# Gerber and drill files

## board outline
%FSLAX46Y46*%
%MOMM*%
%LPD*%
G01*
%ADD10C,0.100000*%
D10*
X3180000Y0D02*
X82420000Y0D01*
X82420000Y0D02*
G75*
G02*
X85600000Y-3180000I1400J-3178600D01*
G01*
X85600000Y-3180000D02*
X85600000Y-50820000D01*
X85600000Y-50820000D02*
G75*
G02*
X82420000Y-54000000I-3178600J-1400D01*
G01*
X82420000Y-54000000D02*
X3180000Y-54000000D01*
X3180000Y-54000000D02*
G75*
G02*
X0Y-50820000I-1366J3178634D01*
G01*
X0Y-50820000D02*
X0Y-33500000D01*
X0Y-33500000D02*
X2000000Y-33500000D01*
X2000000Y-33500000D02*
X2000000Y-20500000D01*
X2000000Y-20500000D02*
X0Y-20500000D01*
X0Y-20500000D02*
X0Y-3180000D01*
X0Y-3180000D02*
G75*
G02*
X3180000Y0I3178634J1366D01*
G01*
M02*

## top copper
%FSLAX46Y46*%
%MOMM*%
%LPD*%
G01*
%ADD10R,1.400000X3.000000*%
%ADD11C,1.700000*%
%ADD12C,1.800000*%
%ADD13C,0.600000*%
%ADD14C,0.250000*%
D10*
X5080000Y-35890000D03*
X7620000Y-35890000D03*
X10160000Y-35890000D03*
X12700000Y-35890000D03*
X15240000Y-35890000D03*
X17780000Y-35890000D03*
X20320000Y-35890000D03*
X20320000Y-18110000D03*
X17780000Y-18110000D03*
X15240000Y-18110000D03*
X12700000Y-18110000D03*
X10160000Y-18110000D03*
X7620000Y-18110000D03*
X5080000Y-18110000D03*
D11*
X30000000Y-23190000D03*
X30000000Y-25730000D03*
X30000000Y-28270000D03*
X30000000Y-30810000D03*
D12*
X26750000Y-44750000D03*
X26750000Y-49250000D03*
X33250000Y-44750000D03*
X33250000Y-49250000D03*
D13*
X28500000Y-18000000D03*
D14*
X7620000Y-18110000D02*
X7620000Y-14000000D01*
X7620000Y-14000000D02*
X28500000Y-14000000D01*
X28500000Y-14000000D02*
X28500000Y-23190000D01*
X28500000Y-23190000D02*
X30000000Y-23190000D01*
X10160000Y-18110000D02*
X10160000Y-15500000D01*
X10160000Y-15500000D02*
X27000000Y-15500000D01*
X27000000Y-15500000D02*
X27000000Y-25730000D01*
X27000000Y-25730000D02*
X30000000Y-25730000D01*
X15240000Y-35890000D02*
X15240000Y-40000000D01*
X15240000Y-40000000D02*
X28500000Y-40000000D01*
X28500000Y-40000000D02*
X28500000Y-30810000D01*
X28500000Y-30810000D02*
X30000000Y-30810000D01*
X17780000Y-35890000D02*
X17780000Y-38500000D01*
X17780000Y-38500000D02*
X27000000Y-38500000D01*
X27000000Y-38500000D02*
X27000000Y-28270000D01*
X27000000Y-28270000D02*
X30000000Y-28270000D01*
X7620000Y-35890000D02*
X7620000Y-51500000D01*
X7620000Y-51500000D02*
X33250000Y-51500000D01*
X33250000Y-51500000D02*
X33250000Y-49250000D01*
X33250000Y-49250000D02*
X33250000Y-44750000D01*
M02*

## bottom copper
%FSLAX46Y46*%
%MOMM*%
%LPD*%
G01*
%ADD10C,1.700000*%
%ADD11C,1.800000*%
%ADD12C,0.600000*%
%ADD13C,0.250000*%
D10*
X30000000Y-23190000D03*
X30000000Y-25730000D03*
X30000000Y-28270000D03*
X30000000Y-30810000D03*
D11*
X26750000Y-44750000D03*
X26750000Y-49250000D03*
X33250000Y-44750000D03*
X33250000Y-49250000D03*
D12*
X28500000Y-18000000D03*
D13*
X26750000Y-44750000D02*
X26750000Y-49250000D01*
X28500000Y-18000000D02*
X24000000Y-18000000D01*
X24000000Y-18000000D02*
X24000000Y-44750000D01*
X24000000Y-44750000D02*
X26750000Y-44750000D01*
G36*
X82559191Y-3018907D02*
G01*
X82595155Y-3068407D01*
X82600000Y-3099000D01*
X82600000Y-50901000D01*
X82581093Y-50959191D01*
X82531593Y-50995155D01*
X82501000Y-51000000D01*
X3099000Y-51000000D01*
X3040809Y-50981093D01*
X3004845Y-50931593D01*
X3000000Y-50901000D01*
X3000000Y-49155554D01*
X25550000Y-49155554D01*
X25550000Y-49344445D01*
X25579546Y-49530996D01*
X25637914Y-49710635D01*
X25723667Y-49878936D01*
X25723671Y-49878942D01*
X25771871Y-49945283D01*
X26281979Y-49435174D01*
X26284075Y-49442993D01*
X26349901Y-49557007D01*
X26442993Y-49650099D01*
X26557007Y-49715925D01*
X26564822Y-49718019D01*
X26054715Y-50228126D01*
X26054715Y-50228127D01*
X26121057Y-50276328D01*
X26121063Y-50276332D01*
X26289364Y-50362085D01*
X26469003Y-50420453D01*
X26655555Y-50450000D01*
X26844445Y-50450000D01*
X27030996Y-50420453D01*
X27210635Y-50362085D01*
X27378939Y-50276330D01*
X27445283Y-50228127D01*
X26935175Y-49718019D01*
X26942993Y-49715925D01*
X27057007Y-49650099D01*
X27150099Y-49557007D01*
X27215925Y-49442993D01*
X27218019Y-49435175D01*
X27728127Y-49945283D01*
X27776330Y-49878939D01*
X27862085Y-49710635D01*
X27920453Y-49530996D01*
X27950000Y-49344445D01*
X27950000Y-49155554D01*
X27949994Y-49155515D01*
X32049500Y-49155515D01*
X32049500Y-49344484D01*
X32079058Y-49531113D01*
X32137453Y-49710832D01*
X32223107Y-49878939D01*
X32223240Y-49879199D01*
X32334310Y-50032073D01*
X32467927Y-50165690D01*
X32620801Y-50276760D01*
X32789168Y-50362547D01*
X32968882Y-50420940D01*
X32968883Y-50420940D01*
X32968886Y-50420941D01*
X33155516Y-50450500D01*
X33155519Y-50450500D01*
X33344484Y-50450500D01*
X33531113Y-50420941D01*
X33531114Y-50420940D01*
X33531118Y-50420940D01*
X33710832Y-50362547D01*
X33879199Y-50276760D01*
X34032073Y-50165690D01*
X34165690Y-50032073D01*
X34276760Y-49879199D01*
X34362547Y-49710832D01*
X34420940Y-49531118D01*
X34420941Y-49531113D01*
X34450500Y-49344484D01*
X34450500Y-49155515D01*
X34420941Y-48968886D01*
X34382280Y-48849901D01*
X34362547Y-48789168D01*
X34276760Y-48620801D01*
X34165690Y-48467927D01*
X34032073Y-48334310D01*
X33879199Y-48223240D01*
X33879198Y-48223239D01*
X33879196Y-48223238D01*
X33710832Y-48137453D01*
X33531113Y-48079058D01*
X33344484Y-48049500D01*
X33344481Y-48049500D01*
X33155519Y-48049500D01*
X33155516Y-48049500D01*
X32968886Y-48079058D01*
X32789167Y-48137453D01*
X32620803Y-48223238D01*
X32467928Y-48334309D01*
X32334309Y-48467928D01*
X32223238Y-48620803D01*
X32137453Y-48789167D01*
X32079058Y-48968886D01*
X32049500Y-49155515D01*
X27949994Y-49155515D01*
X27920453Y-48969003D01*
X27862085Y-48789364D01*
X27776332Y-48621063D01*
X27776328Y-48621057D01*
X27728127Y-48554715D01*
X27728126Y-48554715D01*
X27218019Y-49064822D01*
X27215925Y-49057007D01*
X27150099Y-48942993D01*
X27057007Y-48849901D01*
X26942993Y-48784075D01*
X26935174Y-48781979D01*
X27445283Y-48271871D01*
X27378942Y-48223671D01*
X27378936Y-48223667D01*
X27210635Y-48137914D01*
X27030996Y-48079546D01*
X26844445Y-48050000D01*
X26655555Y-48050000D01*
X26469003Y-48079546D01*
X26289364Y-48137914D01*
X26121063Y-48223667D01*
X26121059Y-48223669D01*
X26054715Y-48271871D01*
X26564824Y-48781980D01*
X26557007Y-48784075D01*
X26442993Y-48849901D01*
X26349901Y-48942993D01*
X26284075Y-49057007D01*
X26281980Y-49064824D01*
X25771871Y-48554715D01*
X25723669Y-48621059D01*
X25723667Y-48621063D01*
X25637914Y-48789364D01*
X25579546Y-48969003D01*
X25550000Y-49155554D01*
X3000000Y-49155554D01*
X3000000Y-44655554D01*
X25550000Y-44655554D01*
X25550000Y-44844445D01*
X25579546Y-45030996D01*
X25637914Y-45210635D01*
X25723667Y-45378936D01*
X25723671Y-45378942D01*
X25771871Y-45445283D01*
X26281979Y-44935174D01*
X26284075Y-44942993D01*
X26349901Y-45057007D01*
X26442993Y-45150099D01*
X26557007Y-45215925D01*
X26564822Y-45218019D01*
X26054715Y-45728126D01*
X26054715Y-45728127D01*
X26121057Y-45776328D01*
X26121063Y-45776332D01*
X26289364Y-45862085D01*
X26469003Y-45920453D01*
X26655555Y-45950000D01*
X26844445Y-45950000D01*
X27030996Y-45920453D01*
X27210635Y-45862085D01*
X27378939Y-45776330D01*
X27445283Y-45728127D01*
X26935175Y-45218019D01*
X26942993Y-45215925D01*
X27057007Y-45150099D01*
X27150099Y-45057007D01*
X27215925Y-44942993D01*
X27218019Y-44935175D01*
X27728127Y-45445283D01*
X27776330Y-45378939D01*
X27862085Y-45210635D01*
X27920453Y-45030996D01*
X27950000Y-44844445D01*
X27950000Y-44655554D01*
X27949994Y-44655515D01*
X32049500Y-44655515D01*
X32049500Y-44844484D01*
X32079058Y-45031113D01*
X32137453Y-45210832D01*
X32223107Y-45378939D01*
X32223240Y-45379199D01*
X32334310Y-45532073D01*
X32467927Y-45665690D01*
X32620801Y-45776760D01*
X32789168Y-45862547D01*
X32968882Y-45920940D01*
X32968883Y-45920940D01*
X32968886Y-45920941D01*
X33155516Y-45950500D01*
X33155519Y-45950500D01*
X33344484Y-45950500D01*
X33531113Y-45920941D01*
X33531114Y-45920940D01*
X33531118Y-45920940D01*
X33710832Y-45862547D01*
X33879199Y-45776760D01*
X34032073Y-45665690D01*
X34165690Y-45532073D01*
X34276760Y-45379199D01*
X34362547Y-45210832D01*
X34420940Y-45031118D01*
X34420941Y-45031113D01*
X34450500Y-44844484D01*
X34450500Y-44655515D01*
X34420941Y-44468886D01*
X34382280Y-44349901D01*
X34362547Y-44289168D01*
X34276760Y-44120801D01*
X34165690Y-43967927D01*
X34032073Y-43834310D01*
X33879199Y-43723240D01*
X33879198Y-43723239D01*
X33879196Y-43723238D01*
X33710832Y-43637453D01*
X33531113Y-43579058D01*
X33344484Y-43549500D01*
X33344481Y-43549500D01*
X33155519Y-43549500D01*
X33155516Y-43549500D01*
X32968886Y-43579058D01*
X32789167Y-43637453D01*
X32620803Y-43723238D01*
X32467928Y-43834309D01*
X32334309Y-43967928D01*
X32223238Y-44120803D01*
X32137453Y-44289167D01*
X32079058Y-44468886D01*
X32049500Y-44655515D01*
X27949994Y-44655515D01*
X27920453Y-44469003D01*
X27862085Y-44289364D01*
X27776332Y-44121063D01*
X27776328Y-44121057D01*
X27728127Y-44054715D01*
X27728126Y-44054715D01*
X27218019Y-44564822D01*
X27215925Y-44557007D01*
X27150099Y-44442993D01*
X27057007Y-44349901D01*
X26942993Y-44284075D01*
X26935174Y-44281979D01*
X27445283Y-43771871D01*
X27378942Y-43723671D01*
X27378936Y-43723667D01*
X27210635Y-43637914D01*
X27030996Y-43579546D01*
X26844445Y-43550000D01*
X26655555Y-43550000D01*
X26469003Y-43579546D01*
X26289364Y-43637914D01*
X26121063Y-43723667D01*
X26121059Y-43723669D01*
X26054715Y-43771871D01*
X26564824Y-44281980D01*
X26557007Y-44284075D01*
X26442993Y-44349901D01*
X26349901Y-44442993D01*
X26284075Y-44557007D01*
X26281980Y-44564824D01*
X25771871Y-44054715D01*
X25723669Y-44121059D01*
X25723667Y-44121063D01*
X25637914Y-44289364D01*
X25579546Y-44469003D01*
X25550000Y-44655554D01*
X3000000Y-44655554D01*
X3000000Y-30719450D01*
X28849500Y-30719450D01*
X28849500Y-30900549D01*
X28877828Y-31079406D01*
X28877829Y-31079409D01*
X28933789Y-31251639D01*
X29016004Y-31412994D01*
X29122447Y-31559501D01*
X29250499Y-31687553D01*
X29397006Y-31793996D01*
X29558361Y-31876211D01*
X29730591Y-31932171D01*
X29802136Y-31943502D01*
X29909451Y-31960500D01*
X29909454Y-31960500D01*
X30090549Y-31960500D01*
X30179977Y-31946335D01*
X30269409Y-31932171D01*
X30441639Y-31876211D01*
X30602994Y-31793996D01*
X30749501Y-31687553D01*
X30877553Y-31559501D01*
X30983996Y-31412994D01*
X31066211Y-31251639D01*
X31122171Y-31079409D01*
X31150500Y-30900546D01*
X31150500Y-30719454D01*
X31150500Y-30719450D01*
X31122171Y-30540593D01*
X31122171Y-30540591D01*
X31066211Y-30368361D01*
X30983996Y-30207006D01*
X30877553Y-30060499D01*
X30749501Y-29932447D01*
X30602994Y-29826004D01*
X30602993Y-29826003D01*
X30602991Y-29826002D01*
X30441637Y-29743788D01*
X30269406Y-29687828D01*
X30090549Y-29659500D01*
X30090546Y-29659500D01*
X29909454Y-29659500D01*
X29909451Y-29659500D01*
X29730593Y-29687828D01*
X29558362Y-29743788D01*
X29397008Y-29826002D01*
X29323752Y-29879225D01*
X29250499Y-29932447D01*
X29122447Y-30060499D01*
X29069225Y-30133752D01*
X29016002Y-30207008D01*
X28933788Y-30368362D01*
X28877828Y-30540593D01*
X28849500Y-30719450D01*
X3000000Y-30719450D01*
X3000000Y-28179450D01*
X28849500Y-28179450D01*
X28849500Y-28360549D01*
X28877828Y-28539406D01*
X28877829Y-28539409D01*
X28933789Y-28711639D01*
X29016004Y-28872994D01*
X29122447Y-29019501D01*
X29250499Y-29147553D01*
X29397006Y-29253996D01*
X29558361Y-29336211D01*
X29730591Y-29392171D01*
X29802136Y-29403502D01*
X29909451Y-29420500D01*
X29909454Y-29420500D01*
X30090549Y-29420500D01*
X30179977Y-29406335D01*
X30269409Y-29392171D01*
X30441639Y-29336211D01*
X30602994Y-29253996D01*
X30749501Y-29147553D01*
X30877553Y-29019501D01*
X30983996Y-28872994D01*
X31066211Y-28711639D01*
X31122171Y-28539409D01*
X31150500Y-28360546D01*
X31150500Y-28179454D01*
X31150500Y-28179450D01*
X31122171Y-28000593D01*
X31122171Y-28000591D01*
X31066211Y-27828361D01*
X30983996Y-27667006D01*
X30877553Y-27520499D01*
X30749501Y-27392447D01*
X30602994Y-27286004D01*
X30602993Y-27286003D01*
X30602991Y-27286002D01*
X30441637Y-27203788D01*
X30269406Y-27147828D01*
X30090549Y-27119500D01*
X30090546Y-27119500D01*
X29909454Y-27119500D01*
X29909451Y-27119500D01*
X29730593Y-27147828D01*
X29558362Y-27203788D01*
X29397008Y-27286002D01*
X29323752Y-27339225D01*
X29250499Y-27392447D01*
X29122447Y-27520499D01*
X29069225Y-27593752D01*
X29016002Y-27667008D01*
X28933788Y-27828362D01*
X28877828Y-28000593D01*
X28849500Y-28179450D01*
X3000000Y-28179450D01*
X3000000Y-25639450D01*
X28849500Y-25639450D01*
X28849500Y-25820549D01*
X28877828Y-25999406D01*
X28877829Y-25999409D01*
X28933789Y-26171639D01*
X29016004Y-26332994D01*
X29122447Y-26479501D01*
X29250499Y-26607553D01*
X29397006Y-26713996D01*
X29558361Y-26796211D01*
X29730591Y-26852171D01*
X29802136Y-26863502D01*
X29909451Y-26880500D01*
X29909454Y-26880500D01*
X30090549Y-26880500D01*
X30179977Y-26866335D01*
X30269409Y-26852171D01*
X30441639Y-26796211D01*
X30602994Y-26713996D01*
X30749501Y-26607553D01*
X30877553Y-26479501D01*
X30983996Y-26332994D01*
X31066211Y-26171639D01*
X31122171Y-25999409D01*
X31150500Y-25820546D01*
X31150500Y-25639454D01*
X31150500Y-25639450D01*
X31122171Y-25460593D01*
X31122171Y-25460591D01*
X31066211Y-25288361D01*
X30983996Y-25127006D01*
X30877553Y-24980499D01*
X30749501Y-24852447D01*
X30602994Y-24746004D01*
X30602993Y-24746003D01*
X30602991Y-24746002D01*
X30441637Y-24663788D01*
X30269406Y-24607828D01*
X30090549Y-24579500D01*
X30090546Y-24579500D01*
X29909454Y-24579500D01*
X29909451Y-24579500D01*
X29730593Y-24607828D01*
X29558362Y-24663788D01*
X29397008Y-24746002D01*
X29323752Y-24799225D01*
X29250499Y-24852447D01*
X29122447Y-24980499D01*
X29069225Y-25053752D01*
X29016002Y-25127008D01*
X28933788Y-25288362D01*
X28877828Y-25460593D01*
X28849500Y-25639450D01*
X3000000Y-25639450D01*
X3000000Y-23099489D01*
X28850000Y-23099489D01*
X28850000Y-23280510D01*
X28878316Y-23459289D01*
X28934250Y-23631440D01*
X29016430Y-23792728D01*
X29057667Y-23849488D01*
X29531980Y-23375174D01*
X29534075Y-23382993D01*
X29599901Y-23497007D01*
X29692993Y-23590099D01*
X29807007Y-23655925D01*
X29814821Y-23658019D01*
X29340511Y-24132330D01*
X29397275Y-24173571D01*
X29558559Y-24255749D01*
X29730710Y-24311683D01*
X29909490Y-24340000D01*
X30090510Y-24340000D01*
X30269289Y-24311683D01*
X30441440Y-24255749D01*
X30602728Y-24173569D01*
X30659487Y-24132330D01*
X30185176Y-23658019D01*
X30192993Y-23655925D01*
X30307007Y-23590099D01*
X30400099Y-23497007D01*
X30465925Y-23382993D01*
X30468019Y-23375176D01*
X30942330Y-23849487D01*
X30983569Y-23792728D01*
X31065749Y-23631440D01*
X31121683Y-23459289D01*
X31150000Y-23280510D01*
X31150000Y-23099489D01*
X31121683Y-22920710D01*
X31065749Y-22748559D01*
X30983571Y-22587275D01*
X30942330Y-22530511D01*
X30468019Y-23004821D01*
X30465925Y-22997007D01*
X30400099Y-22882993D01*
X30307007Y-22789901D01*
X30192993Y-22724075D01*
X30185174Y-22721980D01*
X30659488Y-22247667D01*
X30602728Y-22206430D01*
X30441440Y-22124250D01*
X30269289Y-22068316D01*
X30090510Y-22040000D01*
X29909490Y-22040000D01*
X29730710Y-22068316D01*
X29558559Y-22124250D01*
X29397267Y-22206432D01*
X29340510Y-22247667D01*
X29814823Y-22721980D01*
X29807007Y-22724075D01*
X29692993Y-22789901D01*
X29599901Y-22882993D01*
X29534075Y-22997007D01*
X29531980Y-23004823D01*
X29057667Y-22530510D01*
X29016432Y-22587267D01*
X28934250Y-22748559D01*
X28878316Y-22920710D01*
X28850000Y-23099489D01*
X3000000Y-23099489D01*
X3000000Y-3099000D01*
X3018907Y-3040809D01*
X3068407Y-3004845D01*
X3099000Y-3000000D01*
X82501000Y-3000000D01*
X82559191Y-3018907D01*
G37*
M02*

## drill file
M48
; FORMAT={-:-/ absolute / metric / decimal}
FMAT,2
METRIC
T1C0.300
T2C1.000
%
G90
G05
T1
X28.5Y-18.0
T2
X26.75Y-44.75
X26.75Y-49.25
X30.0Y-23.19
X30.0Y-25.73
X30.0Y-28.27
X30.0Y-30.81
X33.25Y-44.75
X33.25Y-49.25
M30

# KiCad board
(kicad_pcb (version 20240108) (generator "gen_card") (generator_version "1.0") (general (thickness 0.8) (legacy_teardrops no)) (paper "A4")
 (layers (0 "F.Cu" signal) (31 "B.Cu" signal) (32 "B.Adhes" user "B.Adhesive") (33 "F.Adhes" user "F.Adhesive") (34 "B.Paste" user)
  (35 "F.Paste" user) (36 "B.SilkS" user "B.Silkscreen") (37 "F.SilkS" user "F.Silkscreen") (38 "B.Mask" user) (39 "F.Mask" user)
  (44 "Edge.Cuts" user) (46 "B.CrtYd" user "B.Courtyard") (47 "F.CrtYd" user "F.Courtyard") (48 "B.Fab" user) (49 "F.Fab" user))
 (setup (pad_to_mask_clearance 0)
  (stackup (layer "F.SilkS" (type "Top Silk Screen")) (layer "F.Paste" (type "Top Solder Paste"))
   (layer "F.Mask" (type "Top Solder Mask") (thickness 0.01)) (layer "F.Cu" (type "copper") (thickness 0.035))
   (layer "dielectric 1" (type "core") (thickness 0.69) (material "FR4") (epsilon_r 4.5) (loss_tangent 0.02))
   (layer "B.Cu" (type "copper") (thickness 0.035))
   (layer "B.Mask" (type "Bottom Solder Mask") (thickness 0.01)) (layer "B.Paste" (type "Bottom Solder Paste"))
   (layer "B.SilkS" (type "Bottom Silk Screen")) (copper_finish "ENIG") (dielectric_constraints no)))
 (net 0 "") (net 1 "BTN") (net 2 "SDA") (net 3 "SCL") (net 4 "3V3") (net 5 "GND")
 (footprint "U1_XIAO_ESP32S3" (layer "F.Cu") (at 0 0)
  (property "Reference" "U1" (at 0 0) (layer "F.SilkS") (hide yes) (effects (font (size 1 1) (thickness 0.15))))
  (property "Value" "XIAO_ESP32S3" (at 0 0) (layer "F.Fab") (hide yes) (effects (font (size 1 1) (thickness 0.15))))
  (pad "1" smd rect (at 5.080 35.890) (size 1.4 3.0) (layers "F.Cu" "F.Mask" "F.Paste"))
  (pad "2" smd rect (at 7.620 35.890) (size 1.4 3.0) (layers "F.Cu" "F.Mask" "F.Paste") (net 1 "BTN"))
  (pad "3" smd rect (at 10.160 35.890) (size 1.4 3.0) (layers "F.Cu" "F.Mask" "F.Paste"))
  (pad "4" smd rect (at 12.700 35.890) (size 1.4 3.0) (layers "F.Cu" "F.Mask" "F.Paste"))
  (pad "5" smd rect (at 15.240 35.890) (size 1.4 3.0) (layers "F.Cu" "F.Mask" "F.Paste") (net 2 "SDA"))
  (pad "6" smd rect (at 17.780 35.890) (size 1.4 3.0) (layers "F.Cu" "F.Mask" "F.Paste") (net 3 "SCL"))
  (pad "7" smd rect (at 20.320 35.890) (size 1.4 3.0) (layers "F.Cu" "F.Mask" "F.Paste"))
  (pad "8" smd rect (at 20.320 18.110) (size 1.4 3.0) (layers "F.Cu" "F.Mask" "F.Paste"))
  (pad "9" smd rect (at 17.780 18.110) (size 1.4 3.0) (layers "F.Cu" "F.Mask" "F.Paste"))
  (pad "10" smd rect (at 15.240 18.110) (size 1.4 3.0) (layers "F.Cu" "F.Mask" "F.Paste"))
  (pad "11" smd rect (at 12.700 18.110) (size 1.4 3.0) (layers "F.Cu" "F.Mask" "F.Paste"))
  (pad "12" smd rect (at 10.160 18.110) (size 1.4 3.0) (layers "F.Cu" "F.Mask" "F.Paste") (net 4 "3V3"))
  (pad "13" smd rect (at 7.620 18.110) (size 1.4 3.0) (layers "F.Cu" "F.Mask" "F.Paste") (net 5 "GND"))
  (pad "14" smd rect (at 5.080 18.110) (size 1.4 3.0) (layers "F.Cu" "F.Mask" "F.Paste")))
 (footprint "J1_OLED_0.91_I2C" (layer "F.Cu") (at 0 0)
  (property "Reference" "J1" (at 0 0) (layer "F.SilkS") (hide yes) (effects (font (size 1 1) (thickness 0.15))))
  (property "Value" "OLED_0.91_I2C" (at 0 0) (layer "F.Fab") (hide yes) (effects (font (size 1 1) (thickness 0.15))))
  (pad "1" thru_hole circle (at 30.000 23.190) (size 1.7 1.7) (drill 1.0) (layers "*.Cu" "*.Mask") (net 5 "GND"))
  (pad "2" thru_hole circle (at 30.000 25.730) (size 1.7 1.7) (drill 1.0) (layers "*.Cu" "*.Mask") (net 4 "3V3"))
  (pad "3" thru_hole circle (at 30.000 28.270) (size 1.7 1.7) (drill 1.0) (layers "*.Cu" "*.Mask") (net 3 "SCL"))
  (pad "4" thru_hole circle (at 30.000 30.810) (size 1.7 1.7) (drill 1.0) (layers "*.Cu" "*.Mask") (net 2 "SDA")))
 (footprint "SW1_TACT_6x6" (layer "F.Cu") (at 0 0)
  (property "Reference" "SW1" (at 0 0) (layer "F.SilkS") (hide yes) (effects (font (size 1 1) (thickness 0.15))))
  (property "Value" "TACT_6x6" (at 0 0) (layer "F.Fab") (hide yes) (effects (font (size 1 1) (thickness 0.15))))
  (pad "1" thru_hole circle (at 26.750 44.750) (size 1.8 1.8) (drill 1.0) (layers "*.Cu" "*.Mask") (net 5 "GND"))
  (pad "2" thru_hole circle (at 26.750 49.250) (size 1.8 1.8) (drill 1.0) (layers "*.Cu" "*.Mask") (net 5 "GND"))
  (pad "3" thru_hole circle (at 33.250 44.750) (size 1.8 1.8) (drill 1.0) (layers "*.Cu" "*.Mask") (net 1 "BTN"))
  (pad "4" thru_hole circle (at 33.250 49.250) (size 1.8 1.8) (drill 1.0) (layers "*.Cu" "*.Mask") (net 1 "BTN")))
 (segment (start 7.620 18.110) (end 7.620 14.000) (width 0.25) (layer "F.Cu") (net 5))
 (segment (start 7.620 14.000) (end 28.500 14.000) (width 0.25) (layer "F.Cu") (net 5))
 (segment (start 28.500 14.000) (end 28.500 23.190) (width 0.25) (layer "F.Cu") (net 5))
 (segment (start 28.500 23.190) (end 30.000 23.190) (width 0.25) (layer "F.Cu") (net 5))
 (segment (start 10.160 18.110) (end 10.160 15.500) (width 0.25) (layer "F.Cu") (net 4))
 (segment (start 10.160 15.500) (end 27.000 15.500) (width 0.25) (layer "F.Cu") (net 4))
 (segment (start 27.000 15.500) (end 27.000 25.730) (width 0.25) (layer "F.Cu") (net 4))
 (segment (start 27.000 25.730) (end 30.000 25.730) (width 0.25) (layer "F.Cu") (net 4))
 (segment (start 15.240 35.890) (end 15.240 40.000) (width 0.25) (layer "F.Cu") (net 2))
 (segment (start 15.240 40.000) (end 28.500 40.000) (width 0.25) (layer "F.Cu") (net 2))
 (segment (start 28.500 40.000) (end 28.500 30.810) (width 0.25) (layer "F.Cu") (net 2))
 (segment (start 28.500 30.810) (end 30.000 30.810) (width 0.25) (layer "F.Cu") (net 2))
 (segment (start 17.780 35.890) (end 17.780 38.500) (width 0.25) (layer "F.Cu") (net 3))
 (segment (start 17.780 38.500) (end 27.000 38.500) (width 0.25) (layer "F.Cu") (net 3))
 (segment (start 27.000 38.500) (end 27.000 28.270) (width 0.25) (layer "F.Cu") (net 3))
 (segment (start 27.000 28.270) (end 30.000 28.270) (width 0.25) (layer "F.Cu") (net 3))
 (segment (start 7.620 35.890) (end 7.620 51.500) (width 0.25) (layer "F.Cu") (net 1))
 (segment (start 7.620 51.500) (end 33.250 51.500) (width 0.25) (layer "F.Cu") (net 1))
 (segment (start 33.250 51.500) (end 33.250 49.250) (width 0.25) (layer "F.Cu") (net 1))
 (segment (start 33.250 49.250) (end 33.250 44.750) (width 0.25) (layer "F.Cu") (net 1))
 (segment (start 26.750 44.750) (end 26.750 49.250) (width 0.25) (layer "B.Cu") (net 5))
 (via (at 28.500 18.000) (size 0.6) (drill 0.3) (layers "F.Cu" "B.Cu") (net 5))
 (segment (start 28.500 18.000) (end 24.000 18.000) (width 0.25) (layer "B.Cu") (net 5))
 (segment (start 24.000 18.000) (end 24.000 44.750) (width 0.25) (layer "B.Cu") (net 5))
 (segment (start 24.000 44.750) (end 26.750 44.750) (width 0.25) (layer "B.Cu") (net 5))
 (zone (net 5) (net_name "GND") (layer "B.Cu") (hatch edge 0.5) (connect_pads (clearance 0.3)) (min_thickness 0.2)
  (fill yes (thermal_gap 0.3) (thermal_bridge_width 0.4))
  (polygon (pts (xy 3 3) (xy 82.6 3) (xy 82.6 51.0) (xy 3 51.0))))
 (gr_line (start 3.180 0.000) (end 82.420 0.000) (stroke (width 0.1) (type default)) (layer "Edge.Cuts"))
 (gr_arc (start 82.420 0.000) (mid 84.669 0.931) (end 85.600 3.180) (stroke (width 0.1) (type default)) (layer "Edge.Cuts"))
 (gr_line (start 85.600 3.180) (end 85.600 50.820) (stroke (width 0.1) (type default)) (layer "Edge.Cuts"))
 (gr_arc (start 85.600 50.820) (mid 84.669 53.069) (end 82.420 54.000) (stroke (width 0.1) (type default)) (layer "Edge.Cuts"))
 (gr_line (start 82.420 54.000) (end 3.180 54.000) (stroke (width 0.1) (type default)) (layer "Edge.Cuts"))
 (gr_arc (start 3.180 54.000) (mid 0.931 53.069) (end 0.000 50.820) (stroke (width 0.1) (type default)) (layer "Edge.Cuts"))
 (gr_line (start 0.000 50.820) (end 0.000 33.500) (stroke (width 0.1) (type default)) (layer "Edge.Cuts"))
 (gr_line (start 0.000 33.500) (end 2.000 33.500) (stroke (width 0.1) (type default)) (layer "Edge.Cuts"))
 (gr_line (start 2.000 33.500) (end 2.000 20.500) (stroke (width 0.1) (type default)) (layer "Edge.Cuts"))
 (gr_line (start 2.000 20.500) (end 0.000 20.500) (stroke (width 0.1) (type default)) (layer "Edge.Cuts"))
 (gr_line (start 0.000 20.500) (end 0.000 3.180) (stroke (width 0.1) (type default)) (layer "Edge.Cuts"))
 (gr_arc (start 0.000 3.180) (mid 0.931 0.931) (end 3.180 0.000) (stroke (width 0.1) (type default)) (layer "Edge.Cuts")))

